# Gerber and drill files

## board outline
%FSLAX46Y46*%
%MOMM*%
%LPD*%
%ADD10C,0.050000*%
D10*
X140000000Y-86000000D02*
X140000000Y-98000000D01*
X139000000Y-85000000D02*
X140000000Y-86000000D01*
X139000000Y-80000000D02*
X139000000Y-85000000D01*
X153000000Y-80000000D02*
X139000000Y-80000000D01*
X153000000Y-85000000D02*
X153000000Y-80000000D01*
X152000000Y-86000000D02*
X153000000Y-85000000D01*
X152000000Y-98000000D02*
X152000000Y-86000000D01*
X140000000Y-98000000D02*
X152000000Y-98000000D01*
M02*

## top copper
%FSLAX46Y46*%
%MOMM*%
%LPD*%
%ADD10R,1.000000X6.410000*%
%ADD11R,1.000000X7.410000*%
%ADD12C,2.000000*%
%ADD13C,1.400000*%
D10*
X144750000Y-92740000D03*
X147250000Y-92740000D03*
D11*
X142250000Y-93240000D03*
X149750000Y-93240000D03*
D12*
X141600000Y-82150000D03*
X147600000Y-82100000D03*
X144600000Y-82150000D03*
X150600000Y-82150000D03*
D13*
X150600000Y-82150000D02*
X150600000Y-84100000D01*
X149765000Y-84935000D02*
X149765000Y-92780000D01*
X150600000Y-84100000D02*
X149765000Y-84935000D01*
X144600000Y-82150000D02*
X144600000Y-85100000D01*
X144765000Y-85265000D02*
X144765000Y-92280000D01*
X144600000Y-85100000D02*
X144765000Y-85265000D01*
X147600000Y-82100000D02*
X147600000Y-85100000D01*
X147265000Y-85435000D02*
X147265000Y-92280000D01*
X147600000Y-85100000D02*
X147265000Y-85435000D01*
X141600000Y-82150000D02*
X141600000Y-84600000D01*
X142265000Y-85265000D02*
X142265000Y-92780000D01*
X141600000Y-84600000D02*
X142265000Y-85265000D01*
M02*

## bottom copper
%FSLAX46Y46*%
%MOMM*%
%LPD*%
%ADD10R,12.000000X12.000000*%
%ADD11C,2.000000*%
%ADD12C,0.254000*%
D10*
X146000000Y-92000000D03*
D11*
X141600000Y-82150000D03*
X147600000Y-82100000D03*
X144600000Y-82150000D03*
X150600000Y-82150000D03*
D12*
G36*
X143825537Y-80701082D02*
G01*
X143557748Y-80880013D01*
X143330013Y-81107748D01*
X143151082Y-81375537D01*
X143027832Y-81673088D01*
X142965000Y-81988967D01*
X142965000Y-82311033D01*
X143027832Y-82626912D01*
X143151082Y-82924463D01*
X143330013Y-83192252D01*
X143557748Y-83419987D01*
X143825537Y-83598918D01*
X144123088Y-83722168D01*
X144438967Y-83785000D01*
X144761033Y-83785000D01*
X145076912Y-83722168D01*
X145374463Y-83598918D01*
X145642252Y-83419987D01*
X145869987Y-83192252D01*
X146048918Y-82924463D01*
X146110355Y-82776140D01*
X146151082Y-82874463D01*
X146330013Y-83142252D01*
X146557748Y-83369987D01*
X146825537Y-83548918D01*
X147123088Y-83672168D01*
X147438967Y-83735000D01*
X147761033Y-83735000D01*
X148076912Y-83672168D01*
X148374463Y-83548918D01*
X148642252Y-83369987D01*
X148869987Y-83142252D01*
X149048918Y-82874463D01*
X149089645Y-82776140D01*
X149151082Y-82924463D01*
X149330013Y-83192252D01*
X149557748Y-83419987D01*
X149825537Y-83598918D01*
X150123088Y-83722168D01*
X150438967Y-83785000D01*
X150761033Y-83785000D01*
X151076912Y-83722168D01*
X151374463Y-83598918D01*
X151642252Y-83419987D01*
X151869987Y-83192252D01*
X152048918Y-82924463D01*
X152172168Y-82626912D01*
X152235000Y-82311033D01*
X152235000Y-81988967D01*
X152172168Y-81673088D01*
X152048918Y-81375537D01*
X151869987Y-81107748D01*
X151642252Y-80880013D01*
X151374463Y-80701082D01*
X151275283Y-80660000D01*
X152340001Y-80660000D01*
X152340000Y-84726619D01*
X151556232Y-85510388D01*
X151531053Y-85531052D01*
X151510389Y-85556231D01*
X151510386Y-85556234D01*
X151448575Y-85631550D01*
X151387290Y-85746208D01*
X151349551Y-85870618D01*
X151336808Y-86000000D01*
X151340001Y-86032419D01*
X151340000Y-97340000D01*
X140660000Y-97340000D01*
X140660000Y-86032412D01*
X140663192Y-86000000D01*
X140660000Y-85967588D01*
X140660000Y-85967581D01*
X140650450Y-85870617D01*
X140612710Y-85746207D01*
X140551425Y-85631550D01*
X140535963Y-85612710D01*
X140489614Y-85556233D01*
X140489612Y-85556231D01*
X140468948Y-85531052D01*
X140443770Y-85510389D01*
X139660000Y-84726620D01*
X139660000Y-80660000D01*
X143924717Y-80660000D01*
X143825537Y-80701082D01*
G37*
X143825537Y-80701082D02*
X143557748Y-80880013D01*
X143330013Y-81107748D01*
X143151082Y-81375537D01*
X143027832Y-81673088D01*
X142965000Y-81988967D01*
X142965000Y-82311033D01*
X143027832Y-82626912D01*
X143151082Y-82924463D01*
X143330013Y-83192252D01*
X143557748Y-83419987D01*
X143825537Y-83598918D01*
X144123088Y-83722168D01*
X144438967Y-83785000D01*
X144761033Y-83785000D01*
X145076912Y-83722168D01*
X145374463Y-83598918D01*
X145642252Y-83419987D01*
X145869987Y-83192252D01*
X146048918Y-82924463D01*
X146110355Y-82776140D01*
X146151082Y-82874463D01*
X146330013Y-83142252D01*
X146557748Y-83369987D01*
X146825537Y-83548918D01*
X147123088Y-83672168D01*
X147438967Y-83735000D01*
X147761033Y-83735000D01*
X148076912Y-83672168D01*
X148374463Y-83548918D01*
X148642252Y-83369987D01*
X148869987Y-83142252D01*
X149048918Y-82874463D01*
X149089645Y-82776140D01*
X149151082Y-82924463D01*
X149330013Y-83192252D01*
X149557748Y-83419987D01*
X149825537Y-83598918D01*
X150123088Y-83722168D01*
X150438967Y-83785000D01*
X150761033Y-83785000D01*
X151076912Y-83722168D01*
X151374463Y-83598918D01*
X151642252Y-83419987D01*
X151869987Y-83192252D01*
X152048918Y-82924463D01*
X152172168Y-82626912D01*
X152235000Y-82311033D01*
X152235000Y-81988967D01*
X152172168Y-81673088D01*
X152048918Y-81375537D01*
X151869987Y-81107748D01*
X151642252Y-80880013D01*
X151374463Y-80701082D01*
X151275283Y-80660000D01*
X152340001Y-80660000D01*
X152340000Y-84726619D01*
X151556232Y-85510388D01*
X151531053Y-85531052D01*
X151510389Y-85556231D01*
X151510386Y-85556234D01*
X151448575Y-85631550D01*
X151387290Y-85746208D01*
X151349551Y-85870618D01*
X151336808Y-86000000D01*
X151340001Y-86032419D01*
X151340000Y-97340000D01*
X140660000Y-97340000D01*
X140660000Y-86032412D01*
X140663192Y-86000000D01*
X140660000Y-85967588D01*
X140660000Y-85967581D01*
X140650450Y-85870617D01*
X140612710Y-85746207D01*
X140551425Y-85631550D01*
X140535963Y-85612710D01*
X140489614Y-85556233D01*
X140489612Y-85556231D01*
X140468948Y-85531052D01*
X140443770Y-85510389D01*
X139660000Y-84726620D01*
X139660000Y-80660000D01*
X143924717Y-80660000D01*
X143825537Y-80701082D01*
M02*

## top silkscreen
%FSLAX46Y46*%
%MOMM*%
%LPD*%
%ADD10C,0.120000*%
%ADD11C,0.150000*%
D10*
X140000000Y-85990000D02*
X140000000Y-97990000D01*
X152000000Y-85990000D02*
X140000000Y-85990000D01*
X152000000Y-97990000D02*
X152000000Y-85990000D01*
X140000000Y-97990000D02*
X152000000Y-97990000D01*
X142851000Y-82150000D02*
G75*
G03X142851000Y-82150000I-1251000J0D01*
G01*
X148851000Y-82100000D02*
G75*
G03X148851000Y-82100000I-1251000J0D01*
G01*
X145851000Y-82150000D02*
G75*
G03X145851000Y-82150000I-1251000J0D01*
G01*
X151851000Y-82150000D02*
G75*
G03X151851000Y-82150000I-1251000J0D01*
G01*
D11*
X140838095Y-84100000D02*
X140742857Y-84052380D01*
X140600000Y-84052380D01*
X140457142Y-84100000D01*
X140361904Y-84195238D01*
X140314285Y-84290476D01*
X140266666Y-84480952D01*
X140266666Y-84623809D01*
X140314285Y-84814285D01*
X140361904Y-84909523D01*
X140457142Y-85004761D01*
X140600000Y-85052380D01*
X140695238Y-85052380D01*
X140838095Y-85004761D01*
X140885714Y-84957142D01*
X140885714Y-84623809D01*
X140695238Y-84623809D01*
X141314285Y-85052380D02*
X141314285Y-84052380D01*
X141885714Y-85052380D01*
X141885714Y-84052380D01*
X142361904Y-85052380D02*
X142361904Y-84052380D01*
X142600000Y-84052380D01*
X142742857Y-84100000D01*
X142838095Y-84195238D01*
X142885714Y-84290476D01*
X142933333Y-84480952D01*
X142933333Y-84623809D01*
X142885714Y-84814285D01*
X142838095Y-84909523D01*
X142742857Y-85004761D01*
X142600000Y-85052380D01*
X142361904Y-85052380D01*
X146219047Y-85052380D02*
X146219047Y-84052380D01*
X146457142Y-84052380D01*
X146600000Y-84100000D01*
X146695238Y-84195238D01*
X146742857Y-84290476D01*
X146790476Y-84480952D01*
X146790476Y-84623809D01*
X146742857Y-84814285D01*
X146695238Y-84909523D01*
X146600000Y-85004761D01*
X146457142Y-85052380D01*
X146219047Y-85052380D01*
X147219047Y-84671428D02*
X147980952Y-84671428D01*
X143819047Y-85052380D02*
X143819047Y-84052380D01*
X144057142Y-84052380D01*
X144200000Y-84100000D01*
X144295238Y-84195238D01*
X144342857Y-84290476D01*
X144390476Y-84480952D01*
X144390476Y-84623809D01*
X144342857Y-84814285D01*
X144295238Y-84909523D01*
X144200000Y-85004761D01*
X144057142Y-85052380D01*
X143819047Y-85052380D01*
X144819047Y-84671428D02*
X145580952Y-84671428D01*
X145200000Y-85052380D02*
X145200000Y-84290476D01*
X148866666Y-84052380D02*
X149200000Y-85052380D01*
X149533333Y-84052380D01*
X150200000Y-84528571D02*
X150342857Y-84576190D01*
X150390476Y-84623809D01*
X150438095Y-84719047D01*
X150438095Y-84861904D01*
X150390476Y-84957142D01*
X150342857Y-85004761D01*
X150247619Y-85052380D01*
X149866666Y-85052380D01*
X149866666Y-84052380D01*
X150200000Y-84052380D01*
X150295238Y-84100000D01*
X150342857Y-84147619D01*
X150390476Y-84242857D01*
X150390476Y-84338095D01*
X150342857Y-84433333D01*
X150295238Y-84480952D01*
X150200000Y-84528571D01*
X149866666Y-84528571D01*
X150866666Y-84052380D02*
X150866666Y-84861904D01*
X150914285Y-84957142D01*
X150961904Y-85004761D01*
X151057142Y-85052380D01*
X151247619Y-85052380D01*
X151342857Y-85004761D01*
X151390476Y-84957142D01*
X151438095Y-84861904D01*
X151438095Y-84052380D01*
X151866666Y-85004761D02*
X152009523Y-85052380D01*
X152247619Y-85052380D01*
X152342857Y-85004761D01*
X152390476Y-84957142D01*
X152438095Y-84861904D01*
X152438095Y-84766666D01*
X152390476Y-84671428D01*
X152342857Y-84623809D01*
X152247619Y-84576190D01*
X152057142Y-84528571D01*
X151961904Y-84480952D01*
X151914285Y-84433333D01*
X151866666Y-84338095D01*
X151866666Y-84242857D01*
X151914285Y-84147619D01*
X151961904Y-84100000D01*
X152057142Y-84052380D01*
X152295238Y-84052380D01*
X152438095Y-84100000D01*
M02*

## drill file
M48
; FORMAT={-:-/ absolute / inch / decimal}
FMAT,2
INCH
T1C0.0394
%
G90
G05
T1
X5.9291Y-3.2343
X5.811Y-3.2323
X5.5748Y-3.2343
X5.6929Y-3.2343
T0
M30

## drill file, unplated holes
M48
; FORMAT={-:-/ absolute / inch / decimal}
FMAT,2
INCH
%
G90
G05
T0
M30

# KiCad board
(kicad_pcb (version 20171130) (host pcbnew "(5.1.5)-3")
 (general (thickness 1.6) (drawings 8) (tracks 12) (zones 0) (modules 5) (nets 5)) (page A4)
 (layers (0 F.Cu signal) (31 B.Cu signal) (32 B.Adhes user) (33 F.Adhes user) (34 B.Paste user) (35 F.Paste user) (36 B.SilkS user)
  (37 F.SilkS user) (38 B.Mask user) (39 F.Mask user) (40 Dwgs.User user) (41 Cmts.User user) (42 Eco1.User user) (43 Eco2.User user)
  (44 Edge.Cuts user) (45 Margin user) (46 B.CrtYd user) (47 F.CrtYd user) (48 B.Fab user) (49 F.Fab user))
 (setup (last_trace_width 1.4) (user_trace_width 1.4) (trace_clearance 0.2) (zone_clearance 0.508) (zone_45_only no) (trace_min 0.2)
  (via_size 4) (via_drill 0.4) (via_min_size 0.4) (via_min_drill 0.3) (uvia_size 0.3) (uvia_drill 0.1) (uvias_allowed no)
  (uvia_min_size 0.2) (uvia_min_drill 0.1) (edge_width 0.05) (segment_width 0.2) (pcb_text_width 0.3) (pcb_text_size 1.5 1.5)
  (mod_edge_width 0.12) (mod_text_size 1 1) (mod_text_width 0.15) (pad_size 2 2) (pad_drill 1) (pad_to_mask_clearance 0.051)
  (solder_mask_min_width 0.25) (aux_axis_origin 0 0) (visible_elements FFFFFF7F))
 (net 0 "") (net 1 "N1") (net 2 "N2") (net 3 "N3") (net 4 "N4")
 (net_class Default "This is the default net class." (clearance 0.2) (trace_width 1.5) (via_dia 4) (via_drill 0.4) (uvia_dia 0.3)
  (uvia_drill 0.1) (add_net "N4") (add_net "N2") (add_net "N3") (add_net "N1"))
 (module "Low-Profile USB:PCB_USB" (layer F.Cu) (at 146 93.24)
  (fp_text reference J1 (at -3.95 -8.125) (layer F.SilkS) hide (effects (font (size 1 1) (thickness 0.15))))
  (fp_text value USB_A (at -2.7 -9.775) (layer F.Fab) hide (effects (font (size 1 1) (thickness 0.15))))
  (fp_line (start -6 -7.25) (end -6 4.75) (layer F.SilkS) (width 0.12))
  (fp_line (start 6 -7.25) (end -6 -7.25) (layer F.SilkS) (width 0.12))
  (fp_line (start 6 4.75) (end 6 -7.25) (layer F.SilkS) (width 0.12))
  (fp_line (start -6 4.75) (end 6 4.75) (layer F.SilkS) (width 0.12))
  (pad 5 smd rect (at 0 -1.24) (size 12 12) (layers B.Cu B.Paste B.Mask) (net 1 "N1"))
  (pad 3 smd rect (at -1.25 -0.5) (size 1 6.41) (layers F.Cu F.Paste F.Mask) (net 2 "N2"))
  (pad 2 smd rect (at 1.25 -0.5) (size 1 6.41) (layers F.Cu F.Paste F.Mask) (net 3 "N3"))
  (pad 4 smd rect (at -3.75 0) (size 1 7.41) (layers F.Cu F.Paste F.Mask) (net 1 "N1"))
  (pad 1 smd rect (at 3.75 0) (size 1 7.41) (layers F.Cu F.Paste F.Mask) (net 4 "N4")))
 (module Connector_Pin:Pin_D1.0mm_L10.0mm (layer F.Cu) (at 141.6 82.15)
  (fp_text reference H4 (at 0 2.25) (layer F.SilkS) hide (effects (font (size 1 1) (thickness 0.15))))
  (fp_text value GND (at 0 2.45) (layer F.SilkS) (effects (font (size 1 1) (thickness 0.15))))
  (fp_circle (center 0 0) (end 1.25 0.05) (layer F.SilkS) (width 0.12))
  (pad 1 thru_hole circle (at 0 0) (size 2 2) (drill 1) (layers *.Cu *.Mask) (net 1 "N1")))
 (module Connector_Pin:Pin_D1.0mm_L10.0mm (layer F.Cu) (at 147.6 82.1)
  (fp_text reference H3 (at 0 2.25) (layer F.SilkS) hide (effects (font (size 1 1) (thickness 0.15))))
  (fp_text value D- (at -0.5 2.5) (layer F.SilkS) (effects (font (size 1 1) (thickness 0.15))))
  (fp_circle (center 0 0) (end 1.25 0.05) (layer F.SilkS) (width 0.12))
  (pad 1 thru_hole circle (at 0 0) (size 2 2) (drill 1) (layers *.Cu *.Mask) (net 3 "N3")))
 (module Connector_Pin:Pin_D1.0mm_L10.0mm (layer F.Cu) (at 144.6 82.15)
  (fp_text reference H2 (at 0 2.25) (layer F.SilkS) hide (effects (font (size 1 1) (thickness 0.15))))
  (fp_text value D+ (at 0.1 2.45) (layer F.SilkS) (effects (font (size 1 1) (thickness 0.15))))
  (fp_circle (center 0 0) (end 1.25 0.05) (layer F.SilkS) (width 0.12))
  (pad 1 thru_hole circle (at 0 0) (size 2 2) (drill 1) (layers *.Cu *.Mask) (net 2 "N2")))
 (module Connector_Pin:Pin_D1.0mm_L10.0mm (layer F.Cu) (at 150.6 82.15)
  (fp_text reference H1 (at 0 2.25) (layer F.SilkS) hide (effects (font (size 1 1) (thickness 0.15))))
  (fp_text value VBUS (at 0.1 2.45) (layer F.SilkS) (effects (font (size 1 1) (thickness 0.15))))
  (fp_circle (center 0 0) (end 1.25 0.05) (layer F.SilkS) (width 0.12))
  (pad 1 thru_hole circle (at 0 0) (size 2 2) (drill 1) (layers *.Cu *.Mask) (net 4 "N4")))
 (gr_line (start 140 86) (end 140 98) (layer Edge.Cuts) (width 0.05))
 (gr_line (start 139 85) (end 140 86) (layer Edge.Cuts) (width 0.05))
 (gr_line (start 139 80) (end 139 85) (layer Edge.Cuts) (width 0.05))
 (gr_line (start 153 80) (end 139 80) (layer Edge.Cuts) (width 0.05))
 (gr_line (start 153 85) (end 153 80) (layer Edge.Cuts) (width 0.05))
 (gr_line (start 152 86) (end 153 85) (layer Edge.Cuts) (width 0.05))
 (gr_line (start 152 98) (end 152 86) (layer Edge.Cuts) (width 0.05))
 (gr_line (start 140 98) (end 152 98) (layer Edge.Cuts) (width 0.05))
 (segment (start 150.6 82.15) (end 150.6 84.1) (width 1.4) (layer F.Cu) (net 4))
 (segment (start 149.765 84.935) (end 149.765 92.78) (width 1.4) (layer F.Cu) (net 4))
 (segment (start 150.6 84.1) (end 149.765 84.935) (width 1.4) (layer F.Cu) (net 4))
 (segment (start 144.6 82.15) (end 144.6 85.1) (width 1.4) (layer F.Cu) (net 2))
 (segment (start 144.765 85.265) (end 144.765 92.28) (width 1.4) (layer F.Cu) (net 2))
 (segment (start 144.6 85.1) (end 144.765 85.265) (width 1.4) (layer F.Cu) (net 2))
 (segment (start 147.6 82.1) (end 147.6 85.1) (width 1.4) (layer F.Cu) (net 3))
 (segment (start 147.265 85.435) (end 147.265 92.28) (width 1.4) (layer F.Cu) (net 3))
 (segment (start 147.6 85.1) (end 147.265 85.435) (width 1.4) (layer F.Cu) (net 3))
 (segment (start 141.6 82.15) (end 141.6 84.6) (width 1.4) (layer F.Cu) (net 1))
 (segment (start 142.265 85.265) (end 142.265 92.78) (width 1.4) (layer F.Cu) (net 1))
 (segment (start 141.6 84.6) (end 142.265 85.265) (width 1.4) (layer F.Cu) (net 1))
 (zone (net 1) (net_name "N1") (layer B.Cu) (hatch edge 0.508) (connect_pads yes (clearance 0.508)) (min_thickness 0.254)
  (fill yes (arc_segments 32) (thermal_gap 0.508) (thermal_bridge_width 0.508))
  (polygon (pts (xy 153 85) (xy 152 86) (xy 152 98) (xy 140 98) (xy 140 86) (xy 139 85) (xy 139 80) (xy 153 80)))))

